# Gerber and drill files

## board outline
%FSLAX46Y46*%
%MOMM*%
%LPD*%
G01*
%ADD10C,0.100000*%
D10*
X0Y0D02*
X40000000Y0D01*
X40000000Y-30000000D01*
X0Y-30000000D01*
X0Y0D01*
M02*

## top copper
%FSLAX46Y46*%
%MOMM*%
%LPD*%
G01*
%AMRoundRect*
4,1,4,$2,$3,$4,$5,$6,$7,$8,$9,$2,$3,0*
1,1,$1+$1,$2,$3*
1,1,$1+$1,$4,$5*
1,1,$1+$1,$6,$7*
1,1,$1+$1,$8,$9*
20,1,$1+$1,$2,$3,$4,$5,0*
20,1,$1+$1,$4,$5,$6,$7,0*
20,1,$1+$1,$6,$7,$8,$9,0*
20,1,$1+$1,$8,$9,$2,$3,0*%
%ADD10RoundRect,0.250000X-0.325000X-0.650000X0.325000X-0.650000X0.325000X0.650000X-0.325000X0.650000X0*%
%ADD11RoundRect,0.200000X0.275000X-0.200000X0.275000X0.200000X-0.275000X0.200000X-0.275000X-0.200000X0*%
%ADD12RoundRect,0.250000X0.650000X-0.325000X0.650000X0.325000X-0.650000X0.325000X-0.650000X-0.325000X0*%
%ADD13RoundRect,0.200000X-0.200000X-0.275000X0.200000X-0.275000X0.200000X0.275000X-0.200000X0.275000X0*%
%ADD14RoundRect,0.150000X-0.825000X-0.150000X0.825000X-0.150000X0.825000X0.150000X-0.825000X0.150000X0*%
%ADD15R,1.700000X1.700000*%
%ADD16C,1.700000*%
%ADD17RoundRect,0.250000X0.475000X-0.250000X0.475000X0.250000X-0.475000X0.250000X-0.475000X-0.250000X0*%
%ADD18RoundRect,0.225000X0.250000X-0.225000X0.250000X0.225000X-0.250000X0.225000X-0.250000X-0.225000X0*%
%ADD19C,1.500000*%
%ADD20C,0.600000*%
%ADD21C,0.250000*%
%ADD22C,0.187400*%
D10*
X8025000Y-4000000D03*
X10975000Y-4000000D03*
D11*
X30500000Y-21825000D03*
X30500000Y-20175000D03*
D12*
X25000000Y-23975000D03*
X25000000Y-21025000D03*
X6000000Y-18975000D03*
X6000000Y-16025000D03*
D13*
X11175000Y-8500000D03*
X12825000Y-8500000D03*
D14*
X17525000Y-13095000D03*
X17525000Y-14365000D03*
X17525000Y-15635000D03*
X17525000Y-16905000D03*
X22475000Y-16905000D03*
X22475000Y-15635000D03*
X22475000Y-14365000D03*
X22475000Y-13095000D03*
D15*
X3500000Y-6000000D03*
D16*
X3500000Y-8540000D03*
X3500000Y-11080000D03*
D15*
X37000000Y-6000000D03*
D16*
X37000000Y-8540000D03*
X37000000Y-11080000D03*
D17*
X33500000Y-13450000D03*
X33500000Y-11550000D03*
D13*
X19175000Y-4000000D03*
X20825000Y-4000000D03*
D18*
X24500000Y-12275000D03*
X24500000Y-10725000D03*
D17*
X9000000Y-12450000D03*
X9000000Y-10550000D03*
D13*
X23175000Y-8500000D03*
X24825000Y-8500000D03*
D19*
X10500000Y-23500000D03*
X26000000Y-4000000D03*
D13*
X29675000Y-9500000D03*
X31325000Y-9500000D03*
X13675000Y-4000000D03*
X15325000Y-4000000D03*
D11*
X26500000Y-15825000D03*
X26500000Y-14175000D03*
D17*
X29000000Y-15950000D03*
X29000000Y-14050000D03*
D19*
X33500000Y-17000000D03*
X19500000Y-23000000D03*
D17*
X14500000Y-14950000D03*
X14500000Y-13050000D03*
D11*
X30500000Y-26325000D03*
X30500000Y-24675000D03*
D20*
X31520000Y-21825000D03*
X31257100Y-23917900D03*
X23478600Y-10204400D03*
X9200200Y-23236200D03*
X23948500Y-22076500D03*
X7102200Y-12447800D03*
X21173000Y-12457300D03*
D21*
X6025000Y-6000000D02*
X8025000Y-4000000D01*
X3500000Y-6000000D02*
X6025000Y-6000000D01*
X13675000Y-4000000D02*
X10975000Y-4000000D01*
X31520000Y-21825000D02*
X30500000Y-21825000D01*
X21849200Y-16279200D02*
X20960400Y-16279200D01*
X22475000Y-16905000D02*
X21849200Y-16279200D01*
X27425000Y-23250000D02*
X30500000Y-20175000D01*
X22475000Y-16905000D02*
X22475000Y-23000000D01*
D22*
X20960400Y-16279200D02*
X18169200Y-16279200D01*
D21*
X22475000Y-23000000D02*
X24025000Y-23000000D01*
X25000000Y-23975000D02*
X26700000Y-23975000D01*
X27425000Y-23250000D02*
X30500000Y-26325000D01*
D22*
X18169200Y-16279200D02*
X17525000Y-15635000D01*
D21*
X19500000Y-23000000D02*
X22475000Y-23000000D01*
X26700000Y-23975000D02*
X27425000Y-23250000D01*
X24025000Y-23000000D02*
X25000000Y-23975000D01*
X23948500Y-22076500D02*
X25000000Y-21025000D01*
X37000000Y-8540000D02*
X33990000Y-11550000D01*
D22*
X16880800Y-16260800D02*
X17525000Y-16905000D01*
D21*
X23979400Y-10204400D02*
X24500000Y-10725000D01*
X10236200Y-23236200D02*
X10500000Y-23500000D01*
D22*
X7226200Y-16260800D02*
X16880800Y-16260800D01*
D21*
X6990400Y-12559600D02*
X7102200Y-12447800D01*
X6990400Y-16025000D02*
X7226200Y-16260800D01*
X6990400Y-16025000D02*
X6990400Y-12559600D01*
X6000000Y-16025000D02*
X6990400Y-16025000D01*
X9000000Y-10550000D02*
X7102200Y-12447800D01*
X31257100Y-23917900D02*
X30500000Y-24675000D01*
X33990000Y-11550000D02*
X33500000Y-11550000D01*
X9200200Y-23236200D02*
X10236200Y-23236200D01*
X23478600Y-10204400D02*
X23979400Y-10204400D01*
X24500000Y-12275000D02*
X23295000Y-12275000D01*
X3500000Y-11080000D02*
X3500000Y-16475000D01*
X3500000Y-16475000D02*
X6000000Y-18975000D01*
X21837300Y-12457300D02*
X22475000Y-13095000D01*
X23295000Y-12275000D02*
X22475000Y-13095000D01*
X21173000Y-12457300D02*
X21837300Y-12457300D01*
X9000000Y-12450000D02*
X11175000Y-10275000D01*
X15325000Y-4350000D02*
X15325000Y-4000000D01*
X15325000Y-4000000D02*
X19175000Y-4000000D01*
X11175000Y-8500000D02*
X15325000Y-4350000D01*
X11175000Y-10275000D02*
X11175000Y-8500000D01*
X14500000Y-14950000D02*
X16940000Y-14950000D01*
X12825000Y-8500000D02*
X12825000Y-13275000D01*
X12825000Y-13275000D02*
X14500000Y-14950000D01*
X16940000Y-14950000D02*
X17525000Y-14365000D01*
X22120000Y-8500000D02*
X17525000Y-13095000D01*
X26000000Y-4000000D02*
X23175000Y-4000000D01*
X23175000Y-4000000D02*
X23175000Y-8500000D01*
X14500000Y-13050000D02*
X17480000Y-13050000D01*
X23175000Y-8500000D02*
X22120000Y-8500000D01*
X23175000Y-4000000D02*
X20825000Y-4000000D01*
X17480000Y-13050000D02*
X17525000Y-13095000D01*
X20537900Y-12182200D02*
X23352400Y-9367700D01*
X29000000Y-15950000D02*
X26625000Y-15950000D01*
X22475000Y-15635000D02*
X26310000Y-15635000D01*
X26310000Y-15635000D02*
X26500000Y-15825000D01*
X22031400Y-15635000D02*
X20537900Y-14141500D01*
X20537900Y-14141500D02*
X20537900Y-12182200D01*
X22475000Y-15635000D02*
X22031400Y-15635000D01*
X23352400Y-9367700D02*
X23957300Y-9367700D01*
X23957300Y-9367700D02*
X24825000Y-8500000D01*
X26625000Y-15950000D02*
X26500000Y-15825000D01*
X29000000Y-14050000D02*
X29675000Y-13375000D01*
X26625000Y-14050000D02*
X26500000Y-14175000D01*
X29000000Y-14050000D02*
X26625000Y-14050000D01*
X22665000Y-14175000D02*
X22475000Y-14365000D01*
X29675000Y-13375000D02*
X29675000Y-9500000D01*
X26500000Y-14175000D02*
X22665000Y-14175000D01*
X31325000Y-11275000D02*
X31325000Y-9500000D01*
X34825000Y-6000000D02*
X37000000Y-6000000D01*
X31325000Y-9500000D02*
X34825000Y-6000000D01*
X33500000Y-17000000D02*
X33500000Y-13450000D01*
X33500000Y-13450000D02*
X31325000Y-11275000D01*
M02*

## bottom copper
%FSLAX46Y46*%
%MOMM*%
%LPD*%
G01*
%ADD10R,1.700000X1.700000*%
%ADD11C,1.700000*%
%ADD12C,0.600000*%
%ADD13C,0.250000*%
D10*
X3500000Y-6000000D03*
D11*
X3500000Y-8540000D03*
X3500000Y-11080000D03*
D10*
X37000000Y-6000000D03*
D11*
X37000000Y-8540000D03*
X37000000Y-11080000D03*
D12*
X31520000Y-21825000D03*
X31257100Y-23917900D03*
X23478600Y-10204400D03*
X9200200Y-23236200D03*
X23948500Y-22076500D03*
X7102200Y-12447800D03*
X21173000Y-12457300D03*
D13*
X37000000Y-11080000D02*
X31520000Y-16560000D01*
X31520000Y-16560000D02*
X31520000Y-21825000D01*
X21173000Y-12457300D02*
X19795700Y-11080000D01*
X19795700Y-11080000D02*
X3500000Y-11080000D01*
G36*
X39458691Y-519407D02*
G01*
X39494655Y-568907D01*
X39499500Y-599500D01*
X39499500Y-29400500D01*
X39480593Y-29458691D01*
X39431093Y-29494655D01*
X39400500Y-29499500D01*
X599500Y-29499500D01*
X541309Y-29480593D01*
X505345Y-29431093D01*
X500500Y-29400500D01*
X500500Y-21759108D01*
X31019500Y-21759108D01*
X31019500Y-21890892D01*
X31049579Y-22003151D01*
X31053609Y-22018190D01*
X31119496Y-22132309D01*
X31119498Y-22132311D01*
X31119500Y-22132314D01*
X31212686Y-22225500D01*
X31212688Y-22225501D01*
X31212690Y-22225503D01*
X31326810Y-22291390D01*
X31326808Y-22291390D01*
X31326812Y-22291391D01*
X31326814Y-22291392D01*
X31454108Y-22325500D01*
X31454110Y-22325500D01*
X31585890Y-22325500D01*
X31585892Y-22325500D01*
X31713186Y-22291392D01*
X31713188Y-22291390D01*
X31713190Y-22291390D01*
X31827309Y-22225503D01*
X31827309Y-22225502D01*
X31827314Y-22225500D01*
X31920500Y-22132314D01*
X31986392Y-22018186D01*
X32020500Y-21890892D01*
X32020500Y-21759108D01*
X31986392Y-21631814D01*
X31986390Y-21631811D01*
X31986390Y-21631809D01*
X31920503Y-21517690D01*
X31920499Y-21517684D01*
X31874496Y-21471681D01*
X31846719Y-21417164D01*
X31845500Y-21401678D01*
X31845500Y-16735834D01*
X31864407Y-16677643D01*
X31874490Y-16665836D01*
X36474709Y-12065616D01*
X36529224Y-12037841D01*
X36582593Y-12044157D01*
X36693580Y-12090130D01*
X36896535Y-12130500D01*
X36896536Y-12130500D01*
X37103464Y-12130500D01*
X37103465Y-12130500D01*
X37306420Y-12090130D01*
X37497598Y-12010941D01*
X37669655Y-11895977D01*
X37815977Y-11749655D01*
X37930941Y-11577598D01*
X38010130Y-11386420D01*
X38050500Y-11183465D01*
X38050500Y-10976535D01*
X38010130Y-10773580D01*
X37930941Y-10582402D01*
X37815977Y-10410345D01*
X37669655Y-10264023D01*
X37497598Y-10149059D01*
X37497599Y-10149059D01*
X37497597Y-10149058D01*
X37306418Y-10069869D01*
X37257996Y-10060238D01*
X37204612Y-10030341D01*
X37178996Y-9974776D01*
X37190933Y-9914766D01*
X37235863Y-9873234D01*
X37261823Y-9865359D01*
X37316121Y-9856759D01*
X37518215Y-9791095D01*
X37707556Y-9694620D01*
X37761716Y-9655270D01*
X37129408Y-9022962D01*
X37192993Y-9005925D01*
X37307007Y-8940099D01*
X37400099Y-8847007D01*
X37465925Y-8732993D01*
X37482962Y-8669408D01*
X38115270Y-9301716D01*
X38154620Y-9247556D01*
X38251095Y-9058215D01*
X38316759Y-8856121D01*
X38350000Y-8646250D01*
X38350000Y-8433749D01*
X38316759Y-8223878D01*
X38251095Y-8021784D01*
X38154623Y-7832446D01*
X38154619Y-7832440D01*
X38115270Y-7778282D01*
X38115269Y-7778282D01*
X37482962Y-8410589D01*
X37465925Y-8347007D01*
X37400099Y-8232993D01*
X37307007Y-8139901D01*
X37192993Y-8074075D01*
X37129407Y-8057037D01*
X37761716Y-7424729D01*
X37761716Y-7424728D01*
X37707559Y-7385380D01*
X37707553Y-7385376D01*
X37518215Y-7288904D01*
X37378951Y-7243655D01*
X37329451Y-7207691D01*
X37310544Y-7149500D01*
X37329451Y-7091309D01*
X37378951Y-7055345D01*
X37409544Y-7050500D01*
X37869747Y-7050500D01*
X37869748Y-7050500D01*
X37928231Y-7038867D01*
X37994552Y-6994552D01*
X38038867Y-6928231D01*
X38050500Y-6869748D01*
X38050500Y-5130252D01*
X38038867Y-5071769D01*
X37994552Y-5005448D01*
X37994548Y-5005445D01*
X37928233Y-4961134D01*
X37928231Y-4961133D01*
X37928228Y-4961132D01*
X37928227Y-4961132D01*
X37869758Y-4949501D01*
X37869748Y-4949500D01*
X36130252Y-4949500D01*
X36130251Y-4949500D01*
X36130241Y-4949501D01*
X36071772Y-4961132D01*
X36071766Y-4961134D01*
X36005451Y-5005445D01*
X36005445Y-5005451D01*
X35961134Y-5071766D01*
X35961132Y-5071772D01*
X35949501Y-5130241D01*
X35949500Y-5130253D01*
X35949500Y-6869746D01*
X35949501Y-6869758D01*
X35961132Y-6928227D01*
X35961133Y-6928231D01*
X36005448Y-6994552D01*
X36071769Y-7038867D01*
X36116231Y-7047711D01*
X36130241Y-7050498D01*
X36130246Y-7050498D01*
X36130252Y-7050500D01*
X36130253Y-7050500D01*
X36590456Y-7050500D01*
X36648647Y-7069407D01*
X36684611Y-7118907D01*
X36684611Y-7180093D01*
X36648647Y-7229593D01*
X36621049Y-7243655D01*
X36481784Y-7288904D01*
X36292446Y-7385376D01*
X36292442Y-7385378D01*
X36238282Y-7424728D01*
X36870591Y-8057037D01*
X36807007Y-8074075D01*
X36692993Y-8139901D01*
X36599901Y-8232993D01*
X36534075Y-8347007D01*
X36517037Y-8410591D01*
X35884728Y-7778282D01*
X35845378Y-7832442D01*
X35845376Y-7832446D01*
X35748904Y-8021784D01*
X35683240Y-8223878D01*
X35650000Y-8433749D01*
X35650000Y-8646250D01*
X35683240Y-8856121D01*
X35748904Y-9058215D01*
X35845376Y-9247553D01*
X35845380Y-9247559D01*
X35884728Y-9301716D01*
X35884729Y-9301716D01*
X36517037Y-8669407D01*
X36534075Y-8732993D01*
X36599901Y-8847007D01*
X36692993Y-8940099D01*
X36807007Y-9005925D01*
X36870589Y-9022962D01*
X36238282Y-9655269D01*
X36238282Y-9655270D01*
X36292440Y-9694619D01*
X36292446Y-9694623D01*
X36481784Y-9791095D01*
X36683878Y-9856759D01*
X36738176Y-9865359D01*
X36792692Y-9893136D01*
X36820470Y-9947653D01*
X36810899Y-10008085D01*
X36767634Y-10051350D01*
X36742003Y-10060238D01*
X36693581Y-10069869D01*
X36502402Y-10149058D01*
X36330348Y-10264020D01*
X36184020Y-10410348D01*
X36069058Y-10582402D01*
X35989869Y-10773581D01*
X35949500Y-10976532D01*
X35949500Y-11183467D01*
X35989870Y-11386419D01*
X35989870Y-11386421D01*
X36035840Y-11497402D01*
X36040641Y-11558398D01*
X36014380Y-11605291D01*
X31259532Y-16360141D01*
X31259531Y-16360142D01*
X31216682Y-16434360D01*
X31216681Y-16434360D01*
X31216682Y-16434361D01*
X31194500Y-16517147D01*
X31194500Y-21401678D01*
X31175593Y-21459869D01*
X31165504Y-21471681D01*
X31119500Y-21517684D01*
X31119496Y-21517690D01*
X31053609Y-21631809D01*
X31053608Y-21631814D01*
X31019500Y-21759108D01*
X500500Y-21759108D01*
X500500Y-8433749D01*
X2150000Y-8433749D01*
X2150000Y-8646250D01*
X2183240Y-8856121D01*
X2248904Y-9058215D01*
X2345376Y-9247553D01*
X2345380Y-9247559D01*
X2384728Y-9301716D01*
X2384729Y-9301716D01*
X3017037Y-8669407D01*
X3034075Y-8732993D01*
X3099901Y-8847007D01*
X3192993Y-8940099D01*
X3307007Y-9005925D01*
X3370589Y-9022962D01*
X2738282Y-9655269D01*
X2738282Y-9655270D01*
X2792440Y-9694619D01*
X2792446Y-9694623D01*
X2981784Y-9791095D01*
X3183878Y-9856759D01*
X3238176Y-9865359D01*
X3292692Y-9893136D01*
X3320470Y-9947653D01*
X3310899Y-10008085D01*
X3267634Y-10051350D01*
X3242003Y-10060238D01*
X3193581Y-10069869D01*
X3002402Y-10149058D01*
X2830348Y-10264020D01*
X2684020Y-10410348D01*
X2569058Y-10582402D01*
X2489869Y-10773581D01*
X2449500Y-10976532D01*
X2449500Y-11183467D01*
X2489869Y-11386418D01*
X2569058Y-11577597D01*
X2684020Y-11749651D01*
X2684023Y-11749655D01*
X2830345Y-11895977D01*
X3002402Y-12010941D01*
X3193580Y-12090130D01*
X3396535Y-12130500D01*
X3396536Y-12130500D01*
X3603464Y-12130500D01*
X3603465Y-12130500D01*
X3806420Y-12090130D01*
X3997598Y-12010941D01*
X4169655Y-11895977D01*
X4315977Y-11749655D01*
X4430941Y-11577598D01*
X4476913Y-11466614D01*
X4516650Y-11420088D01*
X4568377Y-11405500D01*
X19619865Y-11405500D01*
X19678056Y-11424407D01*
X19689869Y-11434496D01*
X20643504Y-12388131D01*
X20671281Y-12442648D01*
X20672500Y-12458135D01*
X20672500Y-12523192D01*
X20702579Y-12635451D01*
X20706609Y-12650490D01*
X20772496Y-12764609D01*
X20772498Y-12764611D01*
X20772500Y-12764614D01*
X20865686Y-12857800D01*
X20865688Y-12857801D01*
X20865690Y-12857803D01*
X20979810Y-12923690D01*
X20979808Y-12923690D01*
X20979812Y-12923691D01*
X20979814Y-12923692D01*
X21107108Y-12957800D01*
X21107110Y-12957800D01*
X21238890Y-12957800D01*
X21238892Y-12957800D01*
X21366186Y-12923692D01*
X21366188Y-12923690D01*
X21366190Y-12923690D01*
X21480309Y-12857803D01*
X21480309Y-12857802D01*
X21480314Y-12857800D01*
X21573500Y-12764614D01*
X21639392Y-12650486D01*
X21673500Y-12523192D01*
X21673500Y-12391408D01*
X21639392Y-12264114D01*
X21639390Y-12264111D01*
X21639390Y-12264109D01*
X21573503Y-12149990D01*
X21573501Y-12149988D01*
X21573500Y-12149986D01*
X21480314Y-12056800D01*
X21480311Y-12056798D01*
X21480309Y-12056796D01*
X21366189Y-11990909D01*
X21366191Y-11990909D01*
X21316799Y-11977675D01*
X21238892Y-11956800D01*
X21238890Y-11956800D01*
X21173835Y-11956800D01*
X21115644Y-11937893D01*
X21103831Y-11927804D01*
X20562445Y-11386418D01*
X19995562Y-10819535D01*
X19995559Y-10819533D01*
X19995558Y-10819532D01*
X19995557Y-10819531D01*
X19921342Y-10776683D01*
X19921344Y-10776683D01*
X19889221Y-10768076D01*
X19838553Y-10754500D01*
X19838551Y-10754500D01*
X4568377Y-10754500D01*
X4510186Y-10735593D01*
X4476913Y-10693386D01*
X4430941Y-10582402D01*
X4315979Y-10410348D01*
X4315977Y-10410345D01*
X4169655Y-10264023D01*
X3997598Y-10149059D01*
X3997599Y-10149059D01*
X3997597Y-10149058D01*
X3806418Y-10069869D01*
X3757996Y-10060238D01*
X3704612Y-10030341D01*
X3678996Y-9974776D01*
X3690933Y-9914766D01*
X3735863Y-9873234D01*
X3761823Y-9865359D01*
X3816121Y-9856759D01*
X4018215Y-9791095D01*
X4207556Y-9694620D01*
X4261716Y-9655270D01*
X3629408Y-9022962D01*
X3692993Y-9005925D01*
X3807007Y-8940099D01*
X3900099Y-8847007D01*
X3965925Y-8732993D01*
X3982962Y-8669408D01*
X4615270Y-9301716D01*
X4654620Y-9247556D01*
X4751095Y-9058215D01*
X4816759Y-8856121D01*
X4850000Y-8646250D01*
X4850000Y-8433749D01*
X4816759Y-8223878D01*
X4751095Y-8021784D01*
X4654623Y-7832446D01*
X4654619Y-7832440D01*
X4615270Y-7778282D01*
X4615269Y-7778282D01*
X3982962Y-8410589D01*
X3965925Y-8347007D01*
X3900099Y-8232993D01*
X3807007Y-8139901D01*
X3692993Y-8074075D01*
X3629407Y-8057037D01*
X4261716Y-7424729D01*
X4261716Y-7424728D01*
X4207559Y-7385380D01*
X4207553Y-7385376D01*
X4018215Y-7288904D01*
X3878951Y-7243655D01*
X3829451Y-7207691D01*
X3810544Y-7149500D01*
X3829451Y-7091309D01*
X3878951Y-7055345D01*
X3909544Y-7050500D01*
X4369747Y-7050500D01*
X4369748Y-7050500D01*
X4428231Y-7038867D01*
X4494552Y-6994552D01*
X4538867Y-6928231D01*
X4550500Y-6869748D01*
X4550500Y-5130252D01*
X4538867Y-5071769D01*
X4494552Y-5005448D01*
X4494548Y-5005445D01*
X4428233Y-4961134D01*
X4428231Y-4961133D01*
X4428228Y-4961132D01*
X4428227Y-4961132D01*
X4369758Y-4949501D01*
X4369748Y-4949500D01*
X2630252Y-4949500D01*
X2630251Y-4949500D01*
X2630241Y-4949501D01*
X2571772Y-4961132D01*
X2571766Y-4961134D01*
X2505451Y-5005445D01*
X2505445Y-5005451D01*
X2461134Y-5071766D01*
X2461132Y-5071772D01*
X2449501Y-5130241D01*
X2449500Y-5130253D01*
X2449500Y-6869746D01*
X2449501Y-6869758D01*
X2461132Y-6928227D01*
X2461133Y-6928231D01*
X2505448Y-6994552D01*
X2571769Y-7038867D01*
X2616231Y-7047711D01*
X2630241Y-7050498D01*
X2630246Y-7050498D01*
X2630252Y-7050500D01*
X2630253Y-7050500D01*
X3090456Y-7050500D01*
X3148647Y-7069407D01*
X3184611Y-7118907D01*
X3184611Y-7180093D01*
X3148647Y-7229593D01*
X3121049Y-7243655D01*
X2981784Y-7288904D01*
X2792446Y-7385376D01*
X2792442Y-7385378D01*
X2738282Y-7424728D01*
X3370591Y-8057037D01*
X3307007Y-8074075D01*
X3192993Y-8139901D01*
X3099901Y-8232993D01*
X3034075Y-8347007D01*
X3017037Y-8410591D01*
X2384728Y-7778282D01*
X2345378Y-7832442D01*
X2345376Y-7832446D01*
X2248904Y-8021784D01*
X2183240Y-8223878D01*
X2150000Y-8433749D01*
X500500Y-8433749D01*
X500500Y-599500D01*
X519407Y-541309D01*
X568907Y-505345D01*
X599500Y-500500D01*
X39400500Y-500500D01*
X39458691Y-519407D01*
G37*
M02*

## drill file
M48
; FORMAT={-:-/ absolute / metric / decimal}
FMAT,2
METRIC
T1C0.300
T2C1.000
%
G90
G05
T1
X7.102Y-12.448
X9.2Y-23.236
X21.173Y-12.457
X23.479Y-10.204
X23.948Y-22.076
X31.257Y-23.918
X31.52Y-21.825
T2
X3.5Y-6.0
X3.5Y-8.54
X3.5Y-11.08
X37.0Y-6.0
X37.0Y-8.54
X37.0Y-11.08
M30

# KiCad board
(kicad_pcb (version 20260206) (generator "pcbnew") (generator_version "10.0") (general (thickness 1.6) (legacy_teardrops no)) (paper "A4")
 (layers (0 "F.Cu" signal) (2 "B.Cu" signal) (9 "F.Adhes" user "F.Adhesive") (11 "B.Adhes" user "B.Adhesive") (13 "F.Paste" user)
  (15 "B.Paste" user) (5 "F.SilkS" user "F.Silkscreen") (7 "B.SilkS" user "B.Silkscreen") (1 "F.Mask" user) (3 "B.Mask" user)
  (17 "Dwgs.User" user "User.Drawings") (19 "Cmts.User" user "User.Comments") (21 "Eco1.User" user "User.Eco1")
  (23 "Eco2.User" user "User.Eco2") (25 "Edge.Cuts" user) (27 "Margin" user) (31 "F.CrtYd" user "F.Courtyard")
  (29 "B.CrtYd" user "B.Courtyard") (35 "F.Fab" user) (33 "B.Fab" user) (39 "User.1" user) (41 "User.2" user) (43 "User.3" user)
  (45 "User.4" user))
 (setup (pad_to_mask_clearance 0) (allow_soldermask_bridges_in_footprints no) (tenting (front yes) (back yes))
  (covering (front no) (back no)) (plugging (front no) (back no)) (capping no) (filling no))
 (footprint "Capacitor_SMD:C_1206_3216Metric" (layer "F.Cu") (at 9.5 4)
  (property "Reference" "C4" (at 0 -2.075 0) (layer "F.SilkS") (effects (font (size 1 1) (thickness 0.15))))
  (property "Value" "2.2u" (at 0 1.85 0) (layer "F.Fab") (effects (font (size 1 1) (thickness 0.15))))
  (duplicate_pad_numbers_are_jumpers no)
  (pad "1" smd roundrect (at -1.475 0) (size 1.15 1.8) (layers "F.Cu" "F.Mask" "F.Paste") (roundrect_rratio 0.217391) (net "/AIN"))
  (pad "2" smd roundrect (at 1.475 0) (size 1.15 1.8) (layers "F.Cu" "F.Mask" "F.Paste") (roundrect_rratio 0.217391) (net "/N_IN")))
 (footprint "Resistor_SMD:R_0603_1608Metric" (layer "F.Cu") (at 30.5 21 90)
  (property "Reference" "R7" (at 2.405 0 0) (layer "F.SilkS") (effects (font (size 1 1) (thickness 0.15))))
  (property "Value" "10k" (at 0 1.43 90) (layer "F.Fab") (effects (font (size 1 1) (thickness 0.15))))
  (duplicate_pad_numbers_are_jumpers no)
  (pad "1" smd roundrect (at -0.825 0 90) (size 0.8 0.95) (layers "F.Cu" "F.Mask" "F.Paste") (roundrect_rratio 0.25) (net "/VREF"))
  (pad "2" smd roundrect (at 0.825 0 90) (size 0.8 0.95) (layers "F.Cu" "F.Mask" "F.Paste") (roundrect_rratio 0.25) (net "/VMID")))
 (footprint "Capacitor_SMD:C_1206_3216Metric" (layer "F.Cu") (at 25 22.5 90)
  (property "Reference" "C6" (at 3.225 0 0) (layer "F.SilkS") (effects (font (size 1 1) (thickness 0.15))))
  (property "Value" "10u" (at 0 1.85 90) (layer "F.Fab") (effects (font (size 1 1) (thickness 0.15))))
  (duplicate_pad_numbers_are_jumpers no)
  (pad "1" smd roundrect (at -1.475 0 90) (size 1.15 1.8) (layers "F.Cu" "F.Mask" "F.Paste") (roundrect_rratio 0.217391) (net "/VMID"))
  (pad "2" smd roundrect (at 1.475 0 90) (size 1.15 1.8) (layers "F.Cu" "F.Mask" "F.Paste") (roundrect_rratio 0.217391) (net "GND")))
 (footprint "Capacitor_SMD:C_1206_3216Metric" (layer "F.Cu") (at 6 17.5 90)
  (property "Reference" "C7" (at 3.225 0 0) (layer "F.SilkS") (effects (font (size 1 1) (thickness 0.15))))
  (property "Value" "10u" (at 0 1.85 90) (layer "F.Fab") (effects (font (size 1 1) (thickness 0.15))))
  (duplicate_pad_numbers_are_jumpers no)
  (pad "1" smd roundrect (at -1.475 0 90) (size 1.15 1.8) (layers "F.Cu" "F.Mask" "F.Paste") (roundrect_rratio 0.217391) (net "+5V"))
  (pad "2" smd roundrect (at 1.475 0 90) (size 1.15 1.8) (layers "F.Cu" "F.Mask" "F.Paste") (roundrect_rratio 0.217391) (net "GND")))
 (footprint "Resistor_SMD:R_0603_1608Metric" (layer "F.Cu") (at 12 8.5)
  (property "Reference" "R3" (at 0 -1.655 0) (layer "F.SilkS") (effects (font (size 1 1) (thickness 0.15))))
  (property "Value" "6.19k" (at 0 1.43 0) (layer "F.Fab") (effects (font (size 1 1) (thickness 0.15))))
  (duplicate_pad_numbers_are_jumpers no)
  (pad "1" smd roundrect (at -0.825 0) (size 0.8 0.95) (layers "F.Cu" "F.Mask" "F.Paste") (roundrect_rratio 0.25) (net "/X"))
  (pad "2" smd roundrect (at 0.825 0) (size 0.8 0.95) (layers "F.Cu" "F.Mask" "F.Paste") (roundrect_rratio 0.25) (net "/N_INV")))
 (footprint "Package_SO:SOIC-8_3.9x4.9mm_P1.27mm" (layer "F.Cu") (at 20 15)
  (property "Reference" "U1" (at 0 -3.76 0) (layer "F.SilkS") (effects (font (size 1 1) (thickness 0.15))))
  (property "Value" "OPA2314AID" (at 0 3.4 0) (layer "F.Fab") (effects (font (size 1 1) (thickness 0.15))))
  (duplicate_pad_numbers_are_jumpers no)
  (pad "1" smd roundrect (at -2.475 -1.905) (size 1.95 0.6) (layers "F.Cu" "F.Mask" "F.Paste") (roundrect_rratio 0.25) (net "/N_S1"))
  (pad "2" smd roundrect (at -2.475 -0.635) (size 1.95 0.6) (layers "F.Cu" "F.Mask" "F.Paste") (roundrect_rratio 0.25) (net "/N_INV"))
  (pad "3" smd roundrect (at -2.475 0.635) (size 1.95 0.6) (layers "F.Cu" "F.Mask" "F.Paste") (roundrect_rratio 0.25) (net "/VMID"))
  (pad "4" smd roundrect (at -2.475 1.905) (size 1.95 0.6) (layers "F.Cu" "F.Mask" "F.Paste") (roundrect_rratio 0.25) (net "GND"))
  (pad "5" smd roundrect (at 2.475 1.905) (size 1.95 0.6) (layers "F.Cu" "F.Mask" "F.Paste") (roundrect_rratio 0.25) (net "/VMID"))
  (pad "6" smd roundrect (at 2.475 0.635) (size 1.95 0.6) (layers "F.Cu" "F.Mask" "F.Paste") (roundrect_rratio 0.25) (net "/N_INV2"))
  (pad "7" smd roundrect (at 2.475 -0.635) (size 1.95 0.6) (layers "F.Cu" "F.Mask" "F.Paste") (roundrect_rratio 0.25) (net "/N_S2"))
  (pad "8" smd roundrect (at 2.475 -1.905) (size 1.95 0.6) (layers "F.Cu" "F.Mask" "F.Paste") (roundrect_rratio 0.25) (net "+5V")))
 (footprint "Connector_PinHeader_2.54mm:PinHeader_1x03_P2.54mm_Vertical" (layer "F.Cu") (at 3.5 6)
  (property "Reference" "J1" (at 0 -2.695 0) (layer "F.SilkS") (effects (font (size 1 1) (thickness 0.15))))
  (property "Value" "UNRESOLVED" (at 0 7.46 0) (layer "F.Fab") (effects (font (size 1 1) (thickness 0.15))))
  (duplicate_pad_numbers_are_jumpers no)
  (pad "1" thru_hole rect (at 0 0) (size 1.7 1.7) (drill 1) (layers "*.Cu" "*.Mask") (remove_unused_layers no) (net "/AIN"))
  (pad "2" thru_hole circle (at 0 2.54) (size 1.7 1.7) (drill 1) (layers "*.Cu" "*.Mask") (remove_unused_layers no) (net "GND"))
  (pad "3" thru_hole circle (at 0 5.08) (size 1.7 1.7) (drill 1) (layers "*.Cu" "*.Mask") (remove_unused_layers no) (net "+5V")))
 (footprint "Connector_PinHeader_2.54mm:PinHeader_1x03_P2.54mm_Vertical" (layer "F.Cu") (at 37 6)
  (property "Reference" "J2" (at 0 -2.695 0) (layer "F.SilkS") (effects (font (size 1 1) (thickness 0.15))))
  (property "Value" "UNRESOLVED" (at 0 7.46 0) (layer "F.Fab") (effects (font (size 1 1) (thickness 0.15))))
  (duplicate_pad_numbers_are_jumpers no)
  (pad "1" thru_hole rect (at 0 0) (size 1.7 1.7) (drill 1) (layers "*.Cu" "*.Mask") (remove_unused_layers no) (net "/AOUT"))
  (pad "2" thru_hole circle (at 0 2.54) (size 1.7 1.7) (drill 1) (layers "*.Cu" "*.Mask") (remove_unused_layers no) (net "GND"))
  (pad "3" thru_hole circle (at 0 5.08) (size 1.7 1.7) (drill 1) (layers "*.Cu" "*.Mask") (remove_unused_layers no) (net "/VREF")))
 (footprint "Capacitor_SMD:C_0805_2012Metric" (layer "F.Cu") (at 33.5 12.5 90)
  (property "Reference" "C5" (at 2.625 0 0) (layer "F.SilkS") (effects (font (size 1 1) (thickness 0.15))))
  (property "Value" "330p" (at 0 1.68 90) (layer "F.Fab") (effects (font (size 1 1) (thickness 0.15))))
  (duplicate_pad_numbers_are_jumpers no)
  (pad "1" smd roundrect (at -0.95 0 90) (size 1 1.45) (layers "F.Cu" "F.Mask" "F.Paste") (roundrect_rratio 0.25) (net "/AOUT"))
  (pad "2" smd roundrect (at 0.95 0 90) (size 1 1.45) (layers "F.Cu" "F.Mask" "F.Paste") (roundrect_rratio 0.25) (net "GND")))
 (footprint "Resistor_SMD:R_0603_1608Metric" (layer "F.Cu") (at 20 4)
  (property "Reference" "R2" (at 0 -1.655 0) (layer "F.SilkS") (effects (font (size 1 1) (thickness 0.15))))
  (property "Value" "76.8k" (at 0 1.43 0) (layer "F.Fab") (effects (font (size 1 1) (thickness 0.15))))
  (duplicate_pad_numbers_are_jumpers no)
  (pad "1" smd roundrect (at -0.825 0) (size 0.8 0.95) (layers "F.Cu" "F.Mask" "F.Paste") (roundrect_rratio 0.25) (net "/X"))
  (pad "2" smd roundrect (at 0.825 0) (size 0.8 0.95) (layers "F.Cu" "F.Mask" "F.Paste") (roundrect_rratio 0.25) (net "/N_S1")))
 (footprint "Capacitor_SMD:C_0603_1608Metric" (layer "F.Cu") (at 24.5 11.5 90)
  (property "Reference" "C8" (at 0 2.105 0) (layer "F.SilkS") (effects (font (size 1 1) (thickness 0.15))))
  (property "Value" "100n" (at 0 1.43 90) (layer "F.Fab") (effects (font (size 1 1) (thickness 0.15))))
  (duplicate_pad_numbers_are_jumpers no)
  (pad "1" smd roundrect (at -0.775 0 90) (size 0.9 0.95) (layers "F.Cu" "F.Mask" "F.Paste") (roundrect_rratio 0.25) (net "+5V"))
  (pad "2" smd roundrect (at 0.775 0 90) (size 0.9 0.95) (layers "F.Cu" "F.Mask" "F.Paste") (roundrect_rratio 0.25) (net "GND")))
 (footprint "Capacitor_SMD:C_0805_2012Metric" (layer "F.Cu") (at 9 11.5 90)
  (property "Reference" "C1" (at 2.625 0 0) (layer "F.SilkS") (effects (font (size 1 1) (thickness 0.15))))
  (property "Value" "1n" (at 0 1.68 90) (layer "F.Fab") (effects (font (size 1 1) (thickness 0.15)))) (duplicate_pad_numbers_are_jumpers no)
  (pad "1" smd roundrect (at -0.95 0 90) (size 1 1.45) (layers "F.Cu" "F.Mask" "F.Paste") (roundrect_rratio 0.25) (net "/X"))
  (pad "2" smd roundrect (at 0.95 0 90) (size 1 1.45) (layers "F.Cu" "F.Mask" "F.Paste") (roundrect_rratio 0.25) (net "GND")))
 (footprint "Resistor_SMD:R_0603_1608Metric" (layer "F.Cu") (at 24 8.5)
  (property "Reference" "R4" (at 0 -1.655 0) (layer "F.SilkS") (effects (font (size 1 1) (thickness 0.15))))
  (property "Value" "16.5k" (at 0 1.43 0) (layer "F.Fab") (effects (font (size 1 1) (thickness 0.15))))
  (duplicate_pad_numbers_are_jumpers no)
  (pad "1" smd roundrect (at -0.825 0) (size 0.8 0.95) (layers "F.Cu" "F.Mask" "F.Paste") (roundrect_rratio 0.25) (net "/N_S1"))
  (pad "2" smd roundrect (at 0.825 0) (size 0.8 0.95) (layers "F.Cu" "F.Mask" "F.Paste") (roundrect_rratio 0.25) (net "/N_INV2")))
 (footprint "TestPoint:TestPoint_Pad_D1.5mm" (layer "F.Cu") (at 10.5 23.5)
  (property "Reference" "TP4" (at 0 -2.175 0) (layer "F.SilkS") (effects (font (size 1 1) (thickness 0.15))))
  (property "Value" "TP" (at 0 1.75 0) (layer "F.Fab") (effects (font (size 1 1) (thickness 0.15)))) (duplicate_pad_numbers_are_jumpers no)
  (pad "1" smd circle (at 0 0) (size 1.5 1.5) (layers "F.Cu" "F.Mask") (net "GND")))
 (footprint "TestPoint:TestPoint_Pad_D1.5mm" (layer "F.Cu") (at 26 4)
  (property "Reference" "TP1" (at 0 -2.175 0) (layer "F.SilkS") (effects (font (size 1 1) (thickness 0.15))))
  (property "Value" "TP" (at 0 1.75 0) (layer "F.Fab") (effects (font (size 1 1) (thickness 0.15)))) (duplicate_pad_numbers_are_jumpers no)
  (pad "1" smd circle (at 0 0) (size 1.5 1.5) (layers "F.Cu" "F.Mask") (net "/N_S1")))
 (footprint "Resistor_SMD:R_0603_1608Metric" (layer "F.Cu") (at 30.5 9.5)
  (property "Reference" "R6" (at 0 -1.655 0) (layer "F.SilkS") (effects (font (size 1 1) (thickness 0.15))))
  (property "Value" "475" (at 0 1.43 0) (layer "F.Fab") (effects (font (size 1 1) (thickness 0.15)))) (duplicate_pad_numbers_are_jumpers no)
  (pad "1" smd roundrect (at -0.825 0) (size 0.8 0.95) (layers "F.Cu" "F.Mask" "F.Paste") (roundrect_rratio 0.25) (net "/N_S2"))
  (pad "2" smd roundrect (at 0.825 0) (size 0.8 0.95) (layers "F.Cu" "F.Mask" "F.Paste") (roundrect_rratio 0.25) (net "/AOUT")))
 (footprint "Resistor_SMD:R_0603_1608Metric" (layer "F.Cu") (at 14.5 4)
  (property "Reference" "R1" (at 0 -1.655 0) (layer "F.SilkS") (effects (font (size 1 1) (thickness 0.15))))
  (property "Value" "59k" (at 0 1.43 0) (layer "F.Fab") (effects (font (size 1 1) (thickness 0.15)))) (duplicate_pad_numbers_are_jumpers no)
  (pad "1" smd roundrect (at -0.825 0) (size 0.8 0.95) (layers "F.Cu" "F.Mask" "F.Paste") (roundrect_rratio 0.25) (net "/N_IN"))
  (pad "2" smd roundrect (at 0.825 0) (size 0.8 0.95) (layers "F.Cu" "F.Mask" "F.Paste") (roundrect_rratio 0.25) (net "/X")))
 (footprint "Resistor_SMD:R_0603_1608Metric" (layer "F.Cu") (at 26.5 15 90)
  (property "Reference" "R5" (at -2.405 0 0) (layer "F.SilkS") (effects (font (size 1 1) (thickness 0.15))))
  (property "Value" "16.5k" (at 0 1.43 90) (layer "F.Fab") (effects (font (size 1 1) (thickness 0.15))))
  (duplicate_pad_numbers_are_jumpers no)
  (pad "1" smd roundrect (at -0.825 0 90) (size 0.8 0.95) (layers "F.Cu" "F.Mask" "F.Paste") (roundrect_rratio 0.25) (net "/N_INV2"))
  (pad "2" smd roundrect (at 0.825 0 90) (size 0.8 0.95) (layers "F.Cu" "F.Mask" "F.Paste") (roundrect_rratio 0.25) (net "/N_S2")))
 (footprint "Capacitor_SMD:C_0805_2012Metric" (layer "F.Cu") (at 29 15 90)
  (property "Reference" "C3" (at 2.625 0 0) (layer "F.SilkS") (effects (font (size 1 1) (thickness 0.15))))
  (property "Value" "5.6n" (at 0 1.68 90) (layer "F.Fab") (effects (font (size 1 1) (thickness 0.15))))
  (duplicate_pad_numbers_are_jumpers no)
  (pad "1" smd roundrect (at -0.95 0 90) (size 1 1.45) (layers "F.Cu" "F.Mask" "F.Paste") (roundrect_rratio 0.25) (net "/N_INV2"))
  (pad "2" smd roundrect (at 0.95 0 90) (size 1 1.45) (layers "F.Cu" "F.Mask" "F.Paste") (roundrect_rratio 0.25) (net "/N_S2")))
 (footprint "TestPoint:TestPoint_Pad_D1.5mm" (layer "F.Cu") (at 33.5 17)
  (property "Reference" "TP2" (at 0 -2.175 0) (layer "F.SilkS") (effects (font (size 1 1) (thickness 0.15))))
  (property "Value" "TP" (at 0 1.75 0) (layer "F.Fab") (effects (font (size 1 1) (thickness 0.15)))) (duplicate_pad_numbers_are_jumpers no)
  (pad "1" smd circle (at 0 0) (size 1.5 1.5) (layers "F.Cu" "F.Mask") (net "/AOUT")))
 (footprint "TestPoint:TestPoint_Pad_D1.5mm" (layer "F.Cu") (at 19.5 23)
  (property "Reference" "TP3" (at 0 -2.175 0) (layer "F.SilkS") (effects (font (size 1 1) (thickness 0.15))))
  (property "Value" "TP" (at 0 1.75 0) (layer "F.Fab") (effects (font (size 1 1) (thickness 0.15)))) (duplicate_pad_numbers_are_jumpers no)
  (pad "1" smd circle (at 0 0) (size 1.5 1.5) (layers "F.Cu" "F.Mask") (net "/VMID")))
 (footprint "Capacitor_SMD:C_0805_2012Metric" (layer "F.Cu") (at 14.5 14 90)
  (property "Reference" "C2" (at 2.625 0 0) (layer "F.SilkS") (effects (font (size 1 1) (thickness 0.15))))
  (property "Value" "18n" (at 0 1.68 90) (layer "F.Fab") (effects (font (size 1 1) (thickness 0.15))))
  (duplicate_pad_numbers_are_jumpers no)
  (pad "1" smd roundrect (at -0.95 0 90) (size 1 1.45) (layers "F.Cu" "F.Mask" "F.Paste") (roundrect_rratio 0.25) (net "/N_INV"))
  (pad "2" smd roundrect (at 0.95 0 90) (size 1 1.45) (layers "F.Cu" "F.Mask" "F.Paste") (roundrect_rratio 0.25) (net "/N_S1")))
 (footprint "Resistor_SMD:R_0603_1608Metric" (layer "F.Cu") (at 30.5 25.5 90)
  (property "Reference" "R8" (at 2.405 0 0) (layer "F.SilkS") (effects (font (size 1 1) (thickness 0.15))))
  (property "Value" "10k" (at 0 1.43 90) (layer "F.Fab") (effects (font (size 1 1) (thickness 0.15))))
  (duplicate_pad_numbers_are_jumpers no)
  (pad "1" smd roundrect (at -0.825 0 90) (size 0.8 0.95) (layers "F.Cu" "F.Mask" "F.Paste") (roundrect_rratio 0.25) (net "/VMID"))
  (pad "2" smd roundrect (at 0.825 0 90) (size 0.8 0.95) (layers "F.Cu" "F.Mask" "F.Paste") (roundrect_rratio 0.25) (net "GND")))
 (gr_rect (start 0 0) (end 40 30) (stroke (width 0.1) (type default)) (fill no) (layer "Edge.Cuts"))
 (segment (start 6.025 6) (end 8.025 4) (width 0.25) (layer "F.Cu") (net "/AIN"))
 (segment (start 3.5 6) (end 6.025 6) (width 0.25) (layer "F.Cu") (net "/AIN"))
 (segment (start 13.675 4) (end 10.975 4) (width 0.25) (layer "F.Cu") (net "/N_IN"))
 (segment (start 31.52 21.825) (end 30.5 21.825) (width 0.25) (layer "F.Cu") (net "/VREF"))
 (via (at 31.52 21.825) (size 0.6) (drill 0.3) (layers "F.Cu" "B.Cu") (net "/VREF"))
 (segment (start 37 11.08) (end 31.52 16.56) (width 0.25) (layer "B.Cu") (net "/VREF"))
 (segment (start 31.52 16.56) (end 31.52 21.825) (width 0.25) (layer "B.Cu") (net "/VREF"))
 (segment (start 21.8492 16.2792) (end 20.9604 16.2792) (width 0.25) (layer "F.Cu") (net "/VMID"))
 (segment (start 22.475 16.905) (end 21.8492 16.2792) (width 0.25) (layer "F.Cu") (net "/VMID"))
 (segment (start 27.425 23.25) (end 30.5 20.175) (width 0.25) (layer "F.Cu") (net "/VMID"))
 (segment (start 22.475 16.905) (end 22.475 23) (width 0.25) (layer "F.Cu") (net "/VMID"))
 (segment (start 20.9604 16.2792) (end 18.1692 16.2792) (width 0.1874) (layer "F.Cu") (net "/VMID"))
 (segment (start 22.475 23) (end 24.025 23) (width 0.25) (layer "F.Cu") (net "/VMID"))
 (segment (start 25 23.975) (end 26.7 23.975) (width 0.25) (layer "F.Cu") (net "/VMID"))
 (segment (start 27.425 23.25) (end 30.5 26.325) (width 0.25) (layer "F.Cu") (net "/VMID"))
 (segment (start 18.1692 16.2792) (end 17.525 15.635) (width 0.1874) (layer "F.Cu") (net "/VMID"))
 (segment (start 19.5 23) (end 22.475 23) (width 0.25) (layer "F.Cu") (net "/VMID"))
 (segment (start 26.7 23.975) (end 27.425 23.25) (width 0.25) (layer "F.Cu") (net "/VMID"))
 (segment (start 24.025 23) (end 25 23.975) (width 0.25) (layer "F.Cu") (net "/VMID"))
 (segment (start 23.9485 22.0765) (end 25 21.025) (width 0.25) (layer "F.Cu") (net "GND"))
 (segment (start 37 8.54) (end 33.99 11.55) (width 0.25) (layer "F.Cu") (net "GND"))
 (segment (start 16.8808 16.2608) (end 17.525 16.905) (width 0.1874) (layer "F.Cu") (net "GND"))
 (segment (start 23.9794 10.2044) (end 24.5 10.725) (width 0.25) (layer "F.Cu") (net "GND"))
 (segment (start 10.2362 23.2362) (end 10.5 23.5) (width 0.25) (layer "F.Cu") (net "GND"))
 (segment (start 7.2262 16.2608) (end 16.8808 16.2608) (width 0.1874) (layer "F.Cu") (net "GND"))
 (segment (start 6.9904 12.5596) (end 7.1022 12.4478) (width 0.25) (layer "F.Cu") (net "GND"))
 (segment (start 6.9904 16.025) (end 7.2262 16.2608) (width 0.25) (layer "F.Cu") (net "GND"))
 (segment (start 6.9904 16.025) (end 6.9904 12.5596) (width 0.25) (layer "F.Cu") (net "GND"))
 (segment (start 6 16.025) (end 6.9904 16.025) (width 0.25) (layer "F.Cu") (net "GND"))
 (segment (start 9 10.55) (end 7.1022 12.4478) (width 0.25) (layer "F.Cu") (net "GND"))
 (segment (start 31.2571 23.9179) (end 30.5 24.675) (width 0.25) (layer "F.Cu") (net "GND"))
 (segment (start 33.99 11.55) (end 33.5 11.55) (width 0.25) (layer "F.Cu") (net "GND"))
 (segment (start 9.2002 23.2362) (end 10.2362 23.2362) (width 0.25) (layer "F.Cu") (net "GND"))
 (segment (start 23.4786 10.2044) (end 23.9794 10.2044) (width 0.25) (layer "F.Cu") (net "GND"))
 (via (at 31.2571 23.9179) (size 0.6) (drill 0.3) (layers "F.Cu" "B.Cu") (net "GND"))
 (via (at 23.4786 10.2044) (size 0.6) (drill 0.3) (layers "F.Cu" "B.Cu") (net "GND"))
 (via (at 9.2002 23.2362) (size 0.6) (drill 0.3) (layers "F.Cu" "B.Cu") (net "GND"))
 (via (at 23.9485 22.0765) (size 0.6) (drill 0.3) (layers "F.Cu" "B.Cu") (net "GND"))
 (via (at 7.1022 12.4478) (size 0.6) (drill 0.3) (layers "F.Cu" "B.Cu") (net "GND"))
 (segment (start 24.5 12.275) (end 23.295 12.275) (width 0.25) (layer "F.Cu") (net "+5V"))
 (segment (start 3.5 11.08) (end 3.5 16.475) (width 0.25) (layer "F.Cu") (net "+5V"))
 (segment (start 3.5 16.475) (end 6 18.975) (width 0.25) (layer "F.Cu") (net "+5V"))
 (segment (start 21.8373 12.4573) (end 22.475 13.095) (width 0.25) (layer "F.Cu") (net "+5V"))
 (segment (start 23.295 12.275) (end 22.475 13.095) (width 0.25) (layer "F.Cu") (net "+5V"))
 (segment (start 21.173 12.4573) (end 21.8373 12.4573) (width 0.25) (layer "F.Cu") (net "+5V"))
 (via (at 21.173 12.4573) (size 0.6) (drill 0.3) (layers "F.Cu" "B.Cu") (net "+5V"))
 (segment (start 21.173 12.4573) (end 19.7957 11.08) (width 0.25) (layer "B.Cu") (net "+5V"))
 (segment (start 19.7957 11.08) (end 3.5 11.08) (width 0.25) (layer "B.Cu") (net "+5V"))
 (segment (start 9 12.45) (end 11.175 10.275) (width 0.25) (layer "F.Cu") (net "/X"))
 (segment (start 15.325 4.35) (end 15.325 4) (width 0.25) (layer "F.Cu") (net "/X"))
 (segment (start 15.325 4) (end 19.175 4) (width 0.25) (layer "F.Cu") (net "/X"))
 (segment (start 11.175 8.5) (end 15.325 4.35) (width 0.25) (layer "F.Cu") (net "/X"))
 (segment (start 11.175 10.275) (end 11.175 8.5) (width 0.25) (layer "F.Cu") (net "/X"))
 (segment (start 14.5 14.95) (end 16.94 14.95) (width 0.25) (layer "F.Cu") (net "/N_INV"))
 (segment (start 12.825 8.5) (end 12.825 13.275) (width 0.25) (layer "F.Cu") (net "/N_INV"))
 (segment (start 12.825 13.275) (end 14.5 14.95) (width 0.25) (layer "F.Cu") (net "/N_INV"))
 (segment (start 16.94 14.95) (end 17.525 14.365) (width 0.25) (layer "F.Cu") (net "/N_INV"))
 (segment (start 22.12 8.5) (end 17.525 13.095) (width 0.25) (layer "F.Cu") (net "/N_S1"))
 (segment (start 26 4) (end 23.175 4) (width 0.25) (layer "F.Cu") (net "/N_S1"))
 (segment (start 23.175 4) (end 23.175 8.5) (width 0.25) (layer "F.Cu") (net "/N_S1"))
 (segment (start 14.5 13.05) (end 17.48 13.05) (width 0.25) (layer "F.Cu") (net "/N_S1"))
 (segment (start 23.175 8.5) (end 22.12 8.5) (width 0.25) (layer "F.Cu") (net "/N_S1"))
 (segment (start 23.175 4) (end 20.825 4) (width 0.25) (layer "F.Cu") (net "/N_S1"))
 (segment (start 17.48 13.05) (end 17.525 13.095) (width 0.25) (layer "F.Cu") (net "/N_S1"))
 (segment (start 20.5379 12.1822) (end 23.3524 9.3677) (width 0.25) (layer "F.Cu") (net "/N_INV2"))
 (segment (start 29 15.95) (end 26.625 15.95) (width 0.25) (layer "F.Cu") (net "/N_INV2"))
 (segment (start 22.475 15.635) (end 26.31 15.635) (width 0.25) (layer "F.Cu") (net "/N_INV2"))
 (segment (start 26.31 15.635) (end 26.5 15.825) (width 0.25) (layer "F.Cu") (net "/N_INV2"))
 (segment (start 22.0314 15.635) (end 20.5379 14.1415) (width 0.25) (layer "F.Cu") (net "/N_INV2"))
 (segment (start 20.5379 14.1415) (end 20.5379 12.1822) (width 0.25) (layer "F.Cu") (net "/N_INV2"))
 (segment (start 22.475 15.635) (end 22.0314 15.635) (width 0.25) (layer "F.Cu") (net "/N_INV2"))
 (segment (start 23.3524 9.3677) (end 23.9573 9.3677) (width 0.25) (layer "F.Cu") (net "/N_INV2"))
 (segment (start 23.9573 9.3677) (end 24.825 8.5) (width 0.25) (layer "F.Cu") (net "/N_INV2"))
 (segment (start 26.625 15.95) (end 26.5 15.825) (width 0.25) (layer "F.Cu") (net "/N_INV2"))
 (segment (start 29 14.05) (end 29.675 13.375) (width 0.25) (layer "F.Cu") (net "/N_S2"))
 (segment (start 26.625 14.05) (end 26.5 14.175) (width 0.25) (layer "F.Cu") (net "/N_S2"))
 (segment (start 29 14.05) (end 26.625 14.05) (width 0.25) (layer "F.Cu") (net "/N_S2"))
 (segment (start 22.665 14.175) (end 22.475 14.365) (width 0.25) (layer "F.Cu") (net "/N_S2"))
 (segment (start 29.675 13.375) (end 29.675 9.5) (width 0.25) (layer "F.Cu") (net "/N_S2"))
 (segment (start 26.5 14.175) (end 22.665 14.175) (width 0.25) (layer "F.Cu") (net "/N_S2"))
 (segment (start 31.325 11.275) (end 31.325 9.5) (width 0.25) (layer "F.Cu") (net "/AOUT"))
 (segment (start 34.825 6) (end 37 6) (width 0.25) (layer "F.Cu") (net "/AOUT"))
 (segment (start 31.325 9.5) (end 34.825 6) (width 0.25) (layer "F.Cu") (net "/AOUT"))
 (segment (start 33.5 17) (end 33.5 13.45) (width 0.25) (layer "F.Cu") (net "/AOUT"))
 (segment (start 33.5 13.45) (end 31.325 11.275) (width 0.25) (layer "F.Cu") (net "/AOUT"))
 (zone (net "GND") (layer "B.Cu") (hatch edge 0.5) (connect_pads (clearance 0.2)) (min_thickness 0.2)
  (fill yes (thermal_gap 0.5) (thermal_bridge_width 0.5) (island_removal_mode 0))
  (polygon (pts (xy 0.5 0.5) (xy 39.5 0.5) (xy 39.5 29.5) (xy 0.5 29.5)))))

